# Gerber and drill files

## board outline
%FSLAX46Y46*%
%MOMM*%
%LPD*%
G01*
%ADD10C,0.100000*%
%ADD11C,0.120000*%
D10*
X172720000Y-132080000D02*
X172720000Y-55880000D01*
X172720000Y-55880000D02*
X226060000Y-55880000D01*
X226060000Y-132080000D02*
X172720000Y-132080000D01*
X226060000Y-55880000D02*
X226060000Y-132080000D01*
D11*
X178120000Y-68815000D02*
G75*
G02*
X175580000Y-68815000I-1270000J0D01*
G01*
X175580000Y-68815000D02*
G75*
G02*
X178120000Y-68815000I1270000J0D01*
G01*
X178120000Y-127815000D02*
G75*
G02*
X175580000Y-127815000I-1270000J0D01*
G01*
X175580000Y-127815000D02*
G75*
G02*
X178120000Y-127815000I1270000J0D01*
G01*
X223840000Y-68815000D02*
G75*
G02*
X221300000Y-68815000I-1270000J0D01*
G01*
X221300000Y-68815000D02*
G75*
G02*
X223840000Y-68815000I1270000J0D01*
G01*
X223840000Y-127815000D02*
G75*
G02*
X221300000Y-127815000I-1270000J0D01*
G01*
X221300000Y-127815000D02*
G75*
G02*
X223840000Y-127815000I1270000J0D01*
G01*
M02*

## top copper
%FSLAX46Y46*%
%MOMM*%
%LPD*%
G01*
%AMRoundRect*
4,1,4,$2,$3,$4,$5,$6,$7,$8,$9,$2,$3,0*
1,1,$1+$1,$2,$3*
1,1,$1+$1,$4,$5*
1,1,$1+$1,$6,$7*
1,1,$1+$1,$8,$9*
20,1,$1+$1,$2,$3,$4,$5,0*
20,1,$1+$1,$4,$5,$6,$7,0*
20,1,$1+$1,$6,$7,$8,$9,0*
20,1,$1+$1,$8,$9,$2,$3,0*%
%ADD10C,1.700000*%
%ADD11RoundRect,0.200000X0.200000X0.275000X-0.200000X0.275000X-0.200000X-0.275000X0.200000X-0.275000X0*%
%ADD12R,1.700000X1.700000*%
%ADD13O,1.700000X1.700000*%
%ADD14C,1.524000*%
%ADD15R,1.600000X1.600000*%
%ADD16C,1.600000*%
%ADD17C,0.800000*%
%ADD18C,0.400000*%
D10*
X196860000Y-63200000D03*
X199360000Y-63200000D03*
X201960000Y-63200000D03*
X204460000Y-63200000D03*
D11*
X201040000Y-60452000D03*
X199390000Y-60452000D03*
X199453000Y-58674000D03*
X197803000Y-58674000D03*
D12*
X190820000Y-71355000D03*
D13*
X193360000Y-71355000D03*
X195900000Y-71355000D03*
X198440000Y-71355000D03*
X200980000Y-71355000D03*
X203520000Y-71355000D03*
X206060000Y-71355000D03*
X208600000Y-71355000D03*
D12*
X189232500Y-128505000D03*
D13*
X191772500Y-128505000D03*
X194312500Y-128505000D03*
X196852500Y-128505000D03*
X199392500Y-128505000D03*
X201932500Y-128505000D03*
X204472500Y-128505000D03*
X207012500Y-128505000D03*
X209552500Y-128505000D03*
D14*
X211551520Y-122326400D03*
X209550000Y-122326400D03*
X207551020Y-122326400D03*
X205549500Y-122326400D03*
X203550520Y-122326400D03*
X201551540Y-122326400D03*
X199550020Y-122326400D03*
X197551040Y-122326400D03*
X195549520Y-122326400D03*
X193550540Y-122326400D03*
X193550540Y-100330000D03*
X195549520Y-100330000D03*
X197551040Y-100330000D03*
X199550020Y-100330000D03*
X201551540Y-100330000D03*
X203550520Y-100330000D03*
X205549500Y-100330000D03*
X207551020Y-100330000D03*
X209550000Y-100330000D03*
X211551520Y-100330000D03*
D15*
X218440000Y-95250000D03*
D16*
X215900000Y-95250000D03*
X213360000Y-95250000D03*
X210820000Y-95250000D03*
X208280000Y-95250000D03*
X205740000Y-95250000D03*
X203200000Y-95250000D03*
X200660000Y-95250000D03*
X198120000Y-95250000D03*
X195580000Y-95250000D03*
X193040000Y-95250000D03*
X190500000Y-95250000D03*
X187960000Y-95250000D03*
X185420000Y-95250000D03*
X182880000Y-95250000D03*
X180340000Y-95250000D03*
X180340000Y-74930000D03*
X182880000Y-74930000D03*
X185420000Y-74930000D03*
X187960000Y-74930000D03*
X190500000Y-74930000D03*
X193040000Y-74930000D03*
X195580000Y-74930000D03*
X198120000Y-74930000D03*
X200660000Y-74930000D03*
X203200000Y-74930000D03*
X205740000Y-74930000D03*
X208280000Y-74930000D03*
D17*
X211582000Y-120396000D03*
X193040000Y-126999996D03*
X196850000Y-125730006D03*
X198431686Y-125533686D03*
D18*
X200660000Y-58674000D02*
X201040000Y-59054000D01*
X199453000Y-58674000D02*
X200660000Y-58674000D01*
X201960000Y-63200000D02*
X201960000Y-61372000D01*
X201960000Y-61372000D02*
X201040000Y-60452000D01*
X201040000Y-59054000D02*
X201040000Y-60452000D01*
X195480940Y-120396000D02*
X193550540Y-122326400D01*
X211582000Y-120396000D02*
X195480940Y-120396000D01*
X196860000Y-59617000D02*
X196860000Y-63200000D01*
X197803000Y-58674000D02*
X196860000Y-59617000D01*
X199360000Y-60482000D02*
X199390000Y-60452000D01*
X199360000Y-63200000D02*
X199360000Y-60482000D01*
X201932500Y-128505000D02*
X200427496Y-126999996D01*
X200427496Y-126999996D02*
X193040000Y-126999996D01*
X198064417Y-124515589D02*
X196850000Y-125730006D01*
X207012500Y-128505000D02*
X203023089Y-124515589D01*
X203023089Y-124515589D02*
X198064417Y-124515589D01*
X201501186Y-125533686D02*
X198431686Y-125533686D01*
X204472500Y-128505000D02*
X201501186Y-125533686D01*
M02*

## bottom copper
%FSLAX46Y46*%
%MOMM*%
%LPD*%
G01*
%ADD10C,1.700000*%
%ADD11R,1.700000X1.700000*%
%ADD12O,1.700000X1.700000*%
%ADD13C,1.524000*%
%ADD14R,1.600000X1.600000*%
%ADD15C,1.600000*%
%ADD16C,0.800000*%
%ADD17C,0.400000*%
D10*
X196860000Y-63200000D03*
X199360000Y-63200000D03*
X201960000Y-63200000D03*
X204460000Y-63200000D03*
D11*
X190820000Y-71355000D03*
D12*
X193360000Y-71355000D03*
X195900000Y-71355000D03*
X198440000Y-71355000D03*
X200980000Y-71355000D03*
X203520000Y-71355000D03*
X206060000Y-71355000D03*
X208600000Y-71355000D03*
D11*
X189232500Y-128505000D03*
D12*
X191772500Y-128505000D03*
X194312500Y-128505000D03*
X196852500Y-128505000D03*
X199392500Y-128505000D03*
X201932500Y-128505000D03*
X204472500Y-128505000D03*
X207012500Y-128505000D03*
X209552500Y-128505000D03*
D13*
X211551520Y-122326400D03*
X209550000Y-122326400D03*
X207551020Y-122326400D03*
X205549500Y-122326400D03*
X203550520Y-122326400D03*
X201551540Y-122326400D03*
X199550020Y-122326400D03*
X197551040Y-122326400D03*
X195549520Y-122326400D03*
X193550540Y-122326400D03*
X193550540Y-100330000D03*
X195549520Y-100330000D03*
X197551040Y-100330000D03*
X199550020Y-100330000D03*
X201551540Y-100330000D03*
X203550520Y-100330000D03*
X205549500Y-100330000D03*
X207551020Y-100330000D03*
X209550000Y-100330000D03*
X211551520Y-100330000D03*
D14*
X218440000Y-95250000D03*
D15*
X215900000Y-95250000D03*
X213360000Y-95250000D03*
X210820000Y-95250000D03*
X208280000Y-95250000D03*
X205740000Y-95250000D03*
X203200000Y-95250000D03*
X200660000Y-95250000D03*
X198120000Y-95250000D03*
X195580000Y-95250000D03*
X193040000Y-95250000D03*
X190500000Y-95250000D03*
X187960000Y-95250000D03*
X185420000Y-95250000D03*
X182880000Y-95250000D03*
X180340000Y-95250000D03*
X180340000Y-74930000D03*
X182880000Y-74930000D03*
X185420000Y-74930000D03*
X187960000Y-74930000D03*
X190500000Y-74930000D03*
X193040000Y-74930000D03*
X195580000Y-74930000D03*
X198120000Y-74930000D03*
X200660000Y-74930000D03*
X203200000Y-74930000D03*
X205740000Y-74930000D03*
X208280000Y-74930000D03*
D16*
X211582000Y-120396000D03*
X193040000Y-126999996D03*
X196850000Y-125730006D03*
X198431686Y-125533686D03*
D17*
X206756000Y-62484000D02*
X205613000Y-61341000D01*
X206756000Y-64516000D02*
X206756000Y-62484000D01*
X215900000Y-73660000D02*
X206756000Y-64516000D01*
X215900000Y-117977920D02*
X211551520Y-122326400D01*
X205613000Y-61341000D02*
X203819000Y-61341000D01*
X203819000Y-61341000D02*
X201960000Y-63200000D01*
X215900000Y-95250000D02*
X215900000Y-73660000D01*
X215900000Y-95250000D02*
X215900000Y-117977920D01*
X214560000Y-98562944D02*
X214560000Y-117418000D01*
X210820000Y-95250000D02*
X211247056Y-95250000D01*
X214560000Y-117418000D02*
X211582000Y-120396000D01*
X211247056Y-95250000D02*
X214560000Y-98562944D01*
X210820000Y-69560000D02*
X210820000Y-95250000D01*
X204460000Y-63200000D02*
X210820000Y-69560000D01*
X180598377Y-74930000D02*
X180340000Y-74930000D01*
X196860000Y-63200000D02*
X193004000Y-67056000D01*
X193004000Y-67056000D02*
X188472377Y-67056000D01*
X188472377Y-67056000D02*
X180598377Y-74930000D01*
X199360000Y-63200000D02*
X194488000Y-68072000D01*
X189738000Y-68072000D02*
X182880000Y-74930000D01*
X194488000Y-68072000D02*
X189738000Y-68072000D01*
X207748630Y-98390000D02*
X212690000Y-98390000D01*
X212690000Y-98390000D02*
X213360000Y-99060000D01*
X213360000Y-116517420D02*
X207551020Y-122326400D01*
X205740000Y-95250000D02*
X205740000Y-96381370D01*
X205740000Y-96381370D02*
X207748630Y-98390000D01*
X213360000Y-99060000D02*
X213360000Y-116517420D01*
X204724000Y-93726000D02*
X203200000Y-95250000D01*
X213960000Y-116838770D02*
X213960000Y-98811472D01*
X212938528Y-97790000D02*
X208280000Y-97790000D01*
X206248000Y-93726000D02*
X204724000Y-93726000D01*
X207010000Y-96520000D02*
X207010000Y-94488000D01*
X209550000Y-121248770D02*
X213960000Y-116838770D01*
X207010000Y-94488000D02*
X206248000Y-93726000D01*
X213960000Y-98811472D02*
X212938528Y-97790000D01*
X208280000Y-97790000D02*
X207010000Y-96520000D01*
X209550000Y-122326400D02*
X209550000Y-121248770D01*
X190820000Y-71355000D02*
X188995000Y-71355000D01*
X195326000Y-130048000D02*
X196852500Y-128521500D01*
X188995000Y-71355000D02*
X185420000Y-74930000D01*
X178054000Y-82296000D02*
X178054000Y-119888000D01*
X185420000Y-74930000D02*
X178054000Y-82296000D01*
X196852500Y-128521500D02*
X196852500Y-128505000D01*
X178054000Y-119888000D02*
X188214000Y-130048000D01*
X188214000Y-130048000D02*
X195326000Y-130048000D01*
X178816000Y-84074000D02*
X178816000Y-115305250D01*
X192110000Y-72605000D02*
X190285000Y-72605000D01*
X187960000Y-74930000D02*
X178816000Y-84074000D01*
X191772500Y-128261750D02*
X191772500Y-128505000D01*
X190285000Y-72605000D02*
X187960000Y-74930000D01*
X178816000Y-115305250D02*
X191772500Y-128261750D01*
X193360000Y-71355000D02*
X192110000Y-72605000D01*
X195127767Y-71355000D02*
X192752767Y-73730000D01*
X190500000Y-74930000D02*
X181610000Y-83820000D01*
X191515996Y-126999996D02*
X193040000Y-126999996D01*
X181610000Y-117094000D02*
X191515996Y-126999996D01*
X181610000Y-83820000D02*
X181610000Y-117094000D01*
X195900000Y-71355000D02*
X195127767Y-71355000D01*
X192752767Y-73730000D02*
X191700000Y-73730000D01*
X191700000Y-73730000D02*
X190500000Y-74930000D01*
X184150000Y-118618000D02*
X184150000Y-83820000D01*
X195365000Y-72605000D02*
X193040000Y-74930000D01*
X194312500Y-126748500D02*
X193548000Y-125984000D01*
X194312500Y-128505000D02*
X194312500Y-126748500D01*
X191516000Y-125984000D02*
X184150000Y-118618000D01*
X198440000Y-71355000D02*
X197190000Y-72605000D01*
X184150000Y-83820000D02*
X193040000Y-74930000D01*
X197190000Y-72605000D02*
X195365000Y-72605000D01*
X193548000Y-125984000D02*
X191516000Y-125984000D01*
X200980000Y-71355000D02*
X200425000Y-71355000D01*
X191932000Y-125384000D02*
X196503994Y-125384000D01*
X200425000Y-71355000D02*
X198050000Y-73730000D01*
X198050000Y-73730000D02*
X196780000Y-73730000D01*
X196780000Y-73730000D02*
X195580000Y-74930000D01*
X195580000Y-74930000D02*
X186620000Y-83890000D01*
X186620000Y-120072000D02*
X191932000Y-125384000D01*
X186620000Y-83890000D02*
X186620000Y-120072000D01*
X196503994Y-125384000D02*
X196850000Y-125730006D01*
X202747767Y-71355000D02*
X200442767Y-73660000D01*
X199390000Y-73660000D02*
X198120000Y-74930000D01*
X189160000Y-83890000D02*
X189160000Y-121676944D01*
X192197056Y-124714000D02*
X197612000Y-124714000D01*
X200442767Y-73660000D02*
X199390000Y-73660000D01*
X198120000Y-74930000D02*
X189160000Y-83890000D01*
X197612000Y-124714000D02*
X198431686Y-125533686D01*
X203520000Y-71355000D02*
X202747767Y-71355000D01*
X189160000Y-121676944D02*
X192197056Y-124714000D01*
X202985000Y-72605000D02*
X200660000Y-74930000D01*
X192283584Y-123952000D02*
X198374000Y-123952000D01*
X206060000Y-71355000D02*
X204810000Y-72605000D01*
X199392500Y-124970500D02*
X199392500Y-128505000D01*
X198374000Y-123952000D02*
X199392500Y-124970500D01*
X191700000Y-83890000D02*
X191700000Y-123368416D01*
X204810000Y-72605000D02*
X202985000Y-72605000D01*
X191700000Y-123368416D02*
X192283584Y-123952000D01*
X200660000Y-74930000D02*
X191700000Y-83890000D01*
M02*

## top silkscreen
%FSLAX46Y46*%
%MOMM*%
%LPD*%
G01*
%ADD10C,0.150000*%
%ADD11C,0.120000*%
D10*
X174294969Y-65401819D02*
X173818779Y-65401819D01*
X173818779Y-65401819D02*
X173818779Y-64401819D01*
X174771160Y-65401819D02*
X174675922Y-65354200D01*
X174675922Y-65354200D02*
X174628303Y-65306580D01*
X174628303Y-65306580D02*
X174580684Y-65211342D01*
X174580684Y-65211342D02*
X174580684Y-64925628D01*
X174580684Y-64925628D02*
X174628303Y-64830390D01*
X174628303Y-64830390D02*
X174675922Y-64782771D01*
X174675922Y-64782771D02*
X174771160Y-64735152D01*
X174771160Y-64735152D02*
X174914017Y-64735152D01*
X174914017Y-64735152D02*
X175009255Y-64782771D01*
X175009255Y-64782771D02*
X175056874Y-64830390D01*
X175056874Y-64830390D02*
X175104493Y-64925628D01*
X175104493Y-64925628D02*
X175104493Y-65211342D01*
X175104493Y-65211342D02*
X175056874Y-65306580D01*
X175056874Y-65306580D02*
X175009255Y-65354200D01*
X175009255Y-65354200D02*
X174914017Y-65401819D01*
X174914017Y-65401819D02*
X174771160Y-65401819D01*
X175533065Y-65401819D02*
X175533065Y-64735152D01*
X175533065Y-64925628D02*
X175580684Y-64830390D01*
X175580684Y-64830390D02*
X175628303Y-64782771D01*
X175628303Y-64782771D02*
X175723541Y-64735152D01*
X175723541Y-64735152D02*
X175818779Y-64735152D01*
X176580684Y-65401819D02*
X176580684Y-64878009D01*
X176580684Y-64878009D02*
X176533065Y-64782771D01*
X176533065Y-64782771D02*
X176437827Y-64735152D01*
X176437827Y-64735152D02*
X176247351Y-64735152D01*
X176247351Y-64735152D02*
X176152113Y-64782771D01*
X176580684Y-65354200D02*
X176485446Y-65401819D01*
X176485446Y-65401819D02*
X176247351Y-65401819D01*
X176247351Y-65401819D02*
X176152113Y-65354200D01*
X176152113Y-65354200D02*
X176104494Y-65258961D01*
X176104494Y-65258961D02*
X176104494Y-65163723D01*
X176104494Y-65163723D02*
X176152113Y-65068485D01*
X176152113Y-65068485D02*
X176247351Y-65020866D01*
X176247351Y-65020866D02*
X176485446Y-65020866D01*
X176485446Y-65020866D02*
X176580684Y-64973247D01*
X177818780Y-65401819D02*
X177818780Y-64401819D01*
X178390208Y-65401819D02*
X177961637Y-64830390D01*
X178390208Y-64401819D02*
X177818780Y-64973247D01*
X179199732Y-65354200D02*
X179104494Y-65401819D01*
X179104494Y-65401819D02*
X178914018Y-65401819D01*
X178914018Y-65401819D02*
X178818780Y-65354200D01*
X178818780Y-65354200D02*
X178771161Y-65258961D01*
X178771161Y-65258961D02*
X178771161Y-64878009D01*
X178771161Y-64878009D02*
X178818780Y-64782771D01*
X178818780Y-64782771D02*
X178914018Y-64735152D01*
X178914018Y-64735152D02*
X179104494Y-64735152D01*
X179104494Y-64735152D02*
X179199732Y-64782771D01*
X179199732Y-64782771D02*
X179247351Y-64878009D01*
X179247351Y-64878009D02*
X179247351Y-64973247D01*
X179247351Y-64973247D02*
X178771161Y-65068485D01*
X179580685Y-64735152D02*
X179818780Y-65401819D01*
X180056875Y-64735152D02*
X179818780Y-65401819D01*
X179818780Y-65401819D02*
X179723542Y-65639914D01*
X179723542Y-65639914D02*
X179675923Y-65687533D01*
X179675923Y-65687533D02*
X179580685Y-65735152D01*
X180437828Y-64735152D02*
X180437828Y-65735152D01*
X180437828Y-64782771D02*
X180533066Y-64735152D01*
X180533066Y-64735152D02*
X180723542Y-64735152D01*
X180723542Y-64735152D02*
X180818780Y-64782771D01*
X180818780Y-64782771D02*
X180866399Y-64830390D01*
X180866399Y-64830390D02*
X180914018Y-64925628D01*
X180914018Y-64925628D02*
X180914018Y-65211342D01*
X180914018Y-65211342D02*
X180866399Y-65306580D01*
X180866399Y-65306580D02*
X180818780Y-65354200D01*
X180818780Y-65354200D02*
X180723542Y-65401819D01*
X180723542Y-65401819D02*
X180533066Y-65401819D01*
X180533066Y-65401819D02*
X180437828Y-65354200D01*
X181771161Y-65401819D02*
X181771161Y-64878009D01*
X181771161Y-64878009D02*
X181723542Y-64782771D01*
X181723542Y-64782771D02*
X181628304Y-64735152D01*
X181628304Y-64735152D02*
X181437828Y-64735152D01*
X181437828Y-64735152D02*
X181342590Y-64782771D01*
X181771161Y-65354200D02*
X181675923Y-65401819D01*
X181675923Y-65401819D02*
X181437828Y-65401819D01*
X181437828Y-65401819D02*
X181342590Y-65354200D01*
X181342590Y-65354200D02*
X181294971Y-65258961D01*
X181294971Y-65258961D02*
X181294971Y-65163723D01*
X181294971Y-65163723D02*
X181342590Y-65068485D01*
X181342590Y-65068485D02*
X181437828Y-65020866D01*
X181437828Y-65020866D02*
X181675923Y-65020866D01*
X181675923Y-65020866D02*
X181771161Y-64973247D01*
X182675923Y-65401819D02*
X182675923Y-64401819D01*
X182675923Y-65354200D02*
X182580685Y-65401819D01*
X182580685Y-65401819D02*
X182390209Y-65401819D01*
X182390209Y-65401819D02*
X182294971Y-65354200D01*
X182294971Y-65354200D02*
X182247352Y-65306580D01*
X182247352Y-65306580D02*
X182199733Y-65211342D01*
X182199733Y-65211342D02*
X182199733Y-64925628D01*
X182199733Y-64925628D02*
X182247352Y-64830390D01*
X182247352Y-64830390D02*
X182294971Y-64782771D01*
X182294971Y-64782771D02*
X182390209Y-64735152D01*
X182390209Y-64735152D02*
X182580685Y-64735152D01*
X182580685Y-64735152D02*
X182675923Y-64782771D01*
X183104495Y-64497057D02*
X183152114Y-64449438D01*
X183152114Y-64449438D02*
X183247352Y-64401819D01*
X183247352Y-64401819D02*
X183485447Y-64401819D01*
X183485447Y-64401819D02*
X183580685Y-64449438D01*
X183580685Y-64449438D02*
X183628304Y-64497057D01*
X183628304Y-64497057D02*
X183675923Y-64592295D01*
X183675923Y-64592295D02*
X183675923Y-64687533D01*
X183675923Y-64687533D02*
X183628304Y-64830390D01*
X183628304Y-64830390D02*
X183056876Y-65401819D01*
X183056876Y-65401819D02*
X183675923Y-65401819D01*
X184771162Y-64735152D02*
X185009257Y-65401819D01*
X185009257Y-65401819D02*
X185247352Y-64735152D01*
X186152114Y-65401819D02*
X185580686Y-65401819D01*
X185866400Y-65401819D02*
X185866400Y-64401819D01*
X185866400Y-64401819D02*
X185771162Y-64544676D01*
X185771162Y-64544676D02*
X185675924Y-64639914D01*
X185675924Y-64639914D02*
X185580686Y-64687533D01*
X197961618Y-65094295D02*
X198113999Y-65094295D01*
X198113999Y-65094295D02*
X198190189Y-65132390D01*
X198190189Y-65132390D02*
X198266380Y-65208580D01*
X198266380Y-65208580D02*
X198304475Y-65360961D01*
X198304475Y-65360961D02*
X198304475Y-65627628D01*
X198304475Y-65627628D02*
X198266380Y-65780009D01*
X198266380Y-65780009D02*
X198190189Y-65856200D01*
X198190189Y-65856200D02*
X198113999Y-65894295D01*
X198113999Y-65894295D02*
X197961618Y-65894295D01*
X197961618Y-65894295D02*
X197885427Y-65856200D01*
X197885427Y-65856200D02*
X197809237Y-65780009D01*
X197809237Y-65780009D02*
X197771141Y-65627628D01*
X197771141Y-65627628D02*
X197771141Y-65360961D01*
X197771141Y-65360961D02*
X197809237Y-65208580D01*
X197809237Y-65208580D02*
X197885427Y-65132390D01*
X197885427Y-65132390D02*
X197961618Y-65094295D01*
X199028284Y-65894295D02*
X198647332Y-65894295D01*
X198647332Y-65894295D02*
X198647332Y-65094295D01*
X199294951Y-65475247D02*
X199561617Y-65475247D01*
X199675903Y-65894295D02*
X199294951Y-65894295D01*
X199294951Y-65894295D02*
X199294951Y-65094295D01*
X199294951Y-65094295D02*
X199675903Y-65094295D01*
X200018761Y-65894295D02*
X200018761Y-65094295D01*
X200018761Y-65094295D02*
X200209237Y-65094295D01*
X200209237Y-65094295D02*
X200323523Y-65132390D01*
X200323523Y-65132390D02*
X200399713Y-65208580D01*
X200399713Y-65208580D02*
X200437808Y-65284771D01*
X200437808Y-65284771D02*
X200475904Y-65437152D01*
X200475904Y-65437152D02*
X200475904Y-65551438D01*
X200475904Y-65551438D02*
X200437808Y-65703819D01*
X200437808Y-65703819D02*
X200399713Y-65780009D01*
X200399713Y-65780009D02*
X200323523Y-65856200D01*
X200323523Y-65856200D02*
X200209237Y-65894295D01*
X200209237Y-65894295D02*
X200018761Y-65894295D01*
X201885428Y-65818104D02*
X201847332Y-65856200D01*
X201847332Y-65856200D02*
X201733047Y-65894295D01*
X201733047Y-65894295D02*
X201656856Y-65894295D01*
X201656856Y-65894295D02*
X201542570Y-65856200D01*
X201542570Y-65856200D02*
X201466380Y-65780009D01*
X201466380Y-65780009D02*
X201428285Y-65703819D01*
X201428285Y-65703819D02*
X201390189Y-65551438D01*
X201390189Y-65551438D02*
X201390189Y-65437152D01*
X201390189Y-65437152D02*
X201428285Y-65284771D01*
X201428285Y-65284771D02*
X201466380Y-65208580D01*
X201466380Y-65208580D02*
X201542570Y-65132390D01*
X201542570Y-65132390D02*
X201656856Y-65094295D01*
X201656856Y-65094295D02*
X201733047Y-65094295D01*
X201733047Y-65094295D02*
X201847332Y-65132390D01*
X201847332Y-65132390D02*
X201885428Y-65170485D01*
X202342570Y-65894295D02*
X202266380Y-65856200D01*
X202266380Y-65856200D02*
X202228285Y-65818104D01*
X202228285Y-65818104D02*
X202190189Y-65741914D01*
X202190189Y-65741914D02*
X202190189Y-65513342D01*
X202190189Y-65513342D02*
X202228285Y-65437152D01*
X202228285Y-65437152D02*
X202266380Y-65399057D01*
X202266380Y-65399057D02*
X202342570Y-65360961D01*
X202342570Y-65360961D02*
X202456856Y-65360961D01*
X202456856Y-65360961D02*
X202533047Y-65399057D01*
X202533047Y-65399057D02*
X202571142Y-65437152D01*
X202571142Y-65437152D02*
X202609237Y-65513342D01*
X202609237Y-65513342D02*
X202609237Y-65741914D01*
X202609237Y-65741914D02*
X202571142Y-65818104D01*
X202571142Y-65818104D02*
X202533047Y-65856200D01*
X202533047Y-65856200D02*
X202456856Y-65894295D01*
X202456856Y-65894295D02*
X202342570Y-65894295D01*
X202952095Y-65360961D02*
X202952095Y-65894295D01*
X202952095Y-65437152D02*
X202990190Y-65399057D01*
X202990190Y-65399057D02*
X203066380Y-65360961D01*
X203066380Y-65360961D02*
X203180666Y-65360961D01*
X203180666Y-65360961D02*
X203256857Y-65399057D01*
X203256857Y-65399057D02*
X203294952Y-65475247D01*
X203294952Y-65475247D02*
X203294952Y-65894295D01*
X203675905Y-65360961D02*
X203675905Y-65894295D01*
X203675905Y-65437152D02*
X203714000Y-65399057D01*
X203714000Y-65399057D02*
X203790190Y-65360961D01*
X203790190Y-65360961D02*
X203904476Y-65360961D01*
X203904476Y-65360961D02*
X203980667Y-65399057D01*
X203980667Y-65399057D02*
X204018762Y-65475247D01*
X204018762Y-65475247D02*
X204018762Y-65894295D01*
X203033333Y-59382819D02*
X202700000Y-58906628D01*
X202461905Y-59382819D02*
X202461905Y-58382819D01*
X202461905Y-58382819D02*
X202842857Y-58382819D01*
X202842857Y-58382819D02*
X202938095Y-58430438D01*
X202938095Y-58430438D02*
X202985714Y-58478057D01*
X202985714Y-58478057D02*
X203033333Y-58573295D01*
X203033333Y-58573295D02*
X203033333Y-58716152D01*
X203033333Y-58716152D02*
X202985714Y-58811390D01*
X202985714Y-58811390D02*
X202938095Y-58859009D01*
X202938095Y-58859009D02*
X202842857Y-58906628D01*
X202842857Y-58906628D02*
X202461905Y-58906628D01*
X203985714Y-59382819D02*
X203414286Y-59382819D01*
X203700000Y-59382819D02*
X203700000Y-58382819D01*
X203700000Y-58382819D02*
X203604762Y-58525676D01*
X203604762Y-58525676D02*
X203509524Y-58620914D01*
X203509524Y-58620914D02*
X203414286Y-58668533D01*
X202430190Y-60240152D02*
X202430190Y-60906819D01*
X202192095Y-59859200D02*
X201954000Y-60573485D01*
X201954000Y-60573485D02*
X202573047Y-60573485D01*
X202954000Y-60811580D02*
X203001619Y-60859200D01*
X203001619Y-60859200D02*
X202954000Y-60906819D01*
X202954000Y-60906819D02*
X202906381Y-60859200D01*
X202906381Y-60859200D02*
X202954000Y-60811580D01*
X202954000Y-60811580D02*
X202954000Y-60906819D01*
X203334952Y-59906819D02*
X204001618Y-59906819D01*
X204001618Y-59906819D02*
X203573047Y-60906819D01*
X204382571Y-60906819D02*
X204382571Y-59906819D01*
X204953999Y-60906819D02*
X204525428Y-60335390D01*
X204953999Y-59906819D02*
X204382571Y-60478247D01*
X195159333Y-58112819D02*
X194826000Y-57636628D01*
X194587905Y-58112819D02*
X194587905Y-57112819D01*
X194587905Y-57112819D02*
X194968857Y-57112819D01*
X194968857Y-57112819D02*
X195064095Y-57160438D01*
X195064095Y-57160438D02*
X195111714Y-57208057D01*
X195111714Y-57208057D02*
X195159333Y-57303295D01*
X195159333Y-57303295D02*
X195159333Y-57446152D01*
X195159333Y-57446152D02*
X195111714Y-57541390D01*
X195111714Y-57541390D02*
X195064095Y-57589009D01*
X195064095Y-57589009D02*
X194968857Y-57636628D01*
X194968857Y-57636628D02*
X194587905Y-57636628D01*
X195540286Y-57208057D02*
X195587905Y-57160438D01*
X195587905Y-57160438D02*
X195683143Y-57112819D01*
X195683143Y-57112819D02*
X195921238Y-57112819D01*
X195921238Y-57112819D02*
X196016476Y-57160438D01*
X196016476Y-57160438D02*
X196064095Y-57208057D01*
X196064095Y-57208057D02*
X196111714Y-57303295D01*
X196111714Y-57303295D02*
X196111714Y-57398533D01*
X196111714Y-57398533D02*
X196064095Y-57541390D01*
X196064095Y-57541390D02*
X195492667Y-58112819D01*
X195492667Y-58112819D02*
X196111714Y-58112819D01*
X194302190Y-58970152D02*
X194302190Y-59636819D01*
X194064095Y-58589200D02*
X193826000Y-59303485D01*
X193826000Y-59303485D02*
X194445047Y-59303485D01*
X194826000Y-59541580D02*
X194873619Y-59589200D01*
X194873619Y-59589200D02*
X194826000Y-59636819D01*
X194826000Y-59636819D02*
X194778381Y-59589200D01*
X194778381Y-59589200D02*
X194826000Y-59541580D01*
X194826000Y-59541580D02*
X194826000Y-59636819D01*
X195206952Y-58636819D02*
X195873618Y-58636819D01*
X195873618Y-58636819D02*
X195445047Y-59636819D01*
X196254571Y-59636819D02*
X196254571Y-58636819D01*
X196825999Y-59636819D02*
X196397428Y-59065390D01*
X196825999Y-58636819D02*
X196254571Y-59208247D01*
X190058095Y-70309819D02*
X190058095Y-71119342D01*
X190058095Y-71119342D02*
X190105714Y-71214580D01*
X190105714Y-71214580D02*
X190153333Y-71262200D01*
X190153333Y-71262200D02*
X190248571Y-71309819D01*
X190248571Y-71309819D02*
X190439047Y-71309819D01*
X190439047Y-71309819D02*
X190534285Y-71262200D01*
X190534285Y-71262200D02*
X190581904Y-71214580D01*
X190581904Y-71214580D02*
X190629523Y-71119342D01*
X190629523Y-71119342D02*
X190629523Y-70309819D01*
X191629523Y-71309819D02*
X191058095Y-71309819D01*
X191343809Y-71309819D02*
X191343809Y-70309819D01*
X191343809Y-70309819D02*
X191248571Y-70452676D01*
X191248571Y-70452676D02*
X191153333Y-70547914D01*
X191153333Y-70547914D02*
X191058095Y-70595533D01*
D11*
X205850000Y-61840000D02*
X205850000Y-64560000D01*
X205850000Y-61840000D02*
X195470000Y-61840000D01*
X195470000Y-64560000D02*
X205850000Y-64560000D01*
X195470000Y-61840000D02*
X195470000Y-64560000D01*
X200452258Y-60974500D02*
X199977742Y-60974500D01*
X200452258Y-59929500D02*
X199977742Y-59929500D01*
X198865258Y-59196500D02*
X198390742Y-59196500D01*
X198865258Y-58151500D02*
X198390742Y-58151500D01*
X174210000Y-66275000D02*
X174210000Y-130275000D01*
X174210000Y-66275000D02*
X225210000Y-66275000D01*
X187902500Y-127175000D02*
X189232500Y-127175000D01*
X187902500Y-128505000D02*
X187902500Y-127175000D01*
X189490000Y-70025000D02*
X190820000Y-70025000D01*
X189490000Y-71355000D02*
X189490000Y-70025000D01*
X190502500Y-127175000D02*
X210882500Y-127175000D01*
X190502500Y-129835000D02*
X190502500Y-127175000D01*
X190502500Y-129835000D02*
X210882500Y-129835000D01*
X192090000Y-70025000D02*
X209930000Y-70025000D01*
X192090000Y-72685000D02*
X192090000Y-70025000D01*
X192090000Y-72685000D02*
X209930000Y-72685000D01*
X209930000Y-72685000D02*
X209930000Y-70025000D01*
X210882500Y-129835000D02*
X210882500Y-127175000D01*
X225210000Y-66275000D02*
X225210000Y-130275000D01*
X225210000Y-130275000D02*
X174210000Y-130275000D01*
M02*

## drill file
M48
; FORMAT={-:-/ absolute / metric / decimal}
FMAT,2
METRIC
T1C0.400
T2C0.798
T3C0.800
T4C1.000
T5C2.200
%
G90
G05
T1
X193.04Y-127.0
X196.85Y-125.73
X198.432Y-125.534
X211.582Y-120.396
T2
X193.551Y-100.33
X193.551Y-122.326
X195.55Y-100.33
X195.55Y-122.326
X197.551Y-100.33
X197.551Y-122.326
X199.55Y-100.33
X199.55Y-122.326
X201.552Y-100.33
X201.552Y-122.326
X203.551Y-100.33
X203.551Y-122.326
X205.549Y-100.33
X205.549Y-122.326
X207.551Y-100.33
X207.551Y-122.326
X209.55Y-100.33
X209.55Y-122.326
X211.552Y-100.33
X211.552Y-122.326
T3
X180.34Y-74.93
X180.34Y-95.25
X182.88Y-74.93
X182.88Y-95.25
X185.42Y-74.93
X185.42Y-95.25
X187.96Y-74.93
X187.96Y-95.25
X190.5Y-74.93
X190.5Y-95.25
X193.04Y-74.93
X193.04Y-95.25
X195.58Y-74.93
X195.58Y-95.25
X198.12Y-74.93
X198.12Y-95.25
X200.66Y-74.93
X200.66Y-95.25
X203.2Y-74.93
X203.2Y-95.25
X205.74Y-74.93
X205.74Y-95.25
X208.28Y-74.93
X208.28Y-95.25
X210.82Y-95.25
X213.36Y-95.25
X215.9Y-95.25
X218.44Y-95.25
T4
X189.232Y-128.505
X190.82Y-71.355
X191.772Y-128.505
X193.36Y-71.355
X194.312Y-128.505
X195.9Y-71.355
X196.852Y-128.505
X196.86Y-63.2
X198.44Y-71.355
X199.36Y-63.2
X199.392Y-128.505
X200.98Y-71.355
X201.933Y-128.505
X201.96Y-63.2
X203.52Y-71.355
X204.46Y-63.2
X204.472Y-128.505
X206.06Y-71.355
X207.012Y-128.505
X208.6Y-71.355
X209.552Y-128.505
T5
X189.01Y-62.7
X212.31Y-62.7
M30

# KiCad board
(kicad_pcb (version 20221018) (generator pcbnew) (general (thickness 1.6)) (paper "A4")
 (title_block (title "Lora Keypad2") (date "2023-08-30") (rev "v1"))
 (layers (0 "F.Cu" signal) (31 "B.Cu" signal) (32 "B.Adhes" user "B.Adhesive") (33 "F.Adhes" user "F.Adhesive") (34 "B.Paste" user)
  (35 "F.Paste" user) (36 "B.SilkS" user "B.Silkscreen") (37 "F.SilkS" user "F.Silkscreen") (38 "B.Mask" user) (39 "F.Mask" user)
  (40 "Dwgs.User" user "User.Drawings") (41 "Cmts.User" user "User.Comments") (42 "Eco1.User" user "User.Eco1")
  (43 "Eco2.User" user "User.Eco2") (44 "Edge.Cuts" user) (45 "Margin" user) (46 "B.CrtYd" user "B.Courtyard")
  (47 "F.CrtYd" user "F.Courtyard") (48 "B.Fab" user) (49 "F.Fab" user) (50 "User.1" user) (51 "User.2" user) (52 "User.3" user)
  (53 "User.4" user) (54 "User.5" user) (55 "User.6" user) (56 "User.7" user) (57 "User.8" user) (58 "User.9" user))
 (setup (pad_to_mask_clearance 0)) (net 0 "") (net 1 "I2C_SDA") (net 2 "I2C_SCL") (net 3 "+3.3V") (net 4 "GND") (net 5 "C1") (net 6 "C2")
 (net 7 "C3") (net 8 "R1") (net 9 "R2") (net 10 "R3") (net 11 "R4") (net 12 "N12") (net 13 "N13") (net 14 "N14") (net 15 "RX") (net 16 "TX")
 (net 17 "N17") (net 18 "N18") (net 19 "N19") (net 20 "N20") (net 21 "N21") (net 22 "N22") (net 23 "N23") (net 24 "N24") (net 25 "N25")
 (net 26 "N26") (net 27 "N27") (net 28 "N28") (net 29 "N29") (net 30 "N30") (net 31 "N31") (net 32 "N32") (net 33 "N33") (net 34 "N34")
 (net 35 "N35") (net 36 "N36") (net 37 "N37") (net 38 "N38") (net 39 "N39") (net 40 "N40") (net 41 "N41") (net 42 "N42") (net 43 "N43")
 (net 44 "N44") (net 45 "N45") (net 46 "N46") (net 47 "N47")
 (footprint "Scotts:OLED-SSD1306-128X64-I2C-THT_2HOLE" (layer "F.Cu") (at 200.66 63.2 180)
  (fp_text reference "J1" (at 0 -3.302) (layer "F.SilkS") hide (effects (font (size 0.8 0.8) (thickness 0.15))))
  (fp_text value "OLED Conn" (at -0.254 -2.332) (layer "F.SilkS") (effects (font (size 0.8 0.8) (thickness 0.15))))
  (fp_line (start -5.19 1.36) (end -5.19 -1.36) (stroke (width 0.12) (type solid)) (layer "F.SilkS"))
  (fp_line (start -5.19 1.36) (end 5.19 1.36) (stroke (width 0.12) (type solid)) (layer "F.SilkS"))
  (fp_line (start 5.19 -1.36) (end -5.19 -1.36) (stroke (width 0.12) (type solid)) (layer "F.SilkS"))
  (fp_line (start 5.19 1.36) (end 5.19 -1.36) (stroke (width 0.12) (type solid)) (layer "F.SilkS"))
  (pad "" np_thru_hole circle (at -11.65 0.5 180) (size 2.2 2.2) (drill 2.2) (layers "*.Cu" "*.Mask") (solder_mask_margin 1.4)
   (clearance 1.4))
  (pad "" np_thru_hole circle (at 11.65 0.5 180) (size 2.2 2.2) (drill 2.2) (layers "*.Cu" "*.Mask") (solder_mask_margin 1.4)
   (clearance 1.4))
  (pad "1" thru_hole circle (at 3.8 0 180) (size 1.7 1.7) (drill 1) (layers "*.Cu" "*.Mask") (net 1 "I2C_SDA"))
  (pad "2" thru_hole circle (at 1.3 0 180) (size 1.7 1.7) (drill 1) (layers "*.Cu" "*.Mask") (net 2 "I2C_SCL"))
  (pad "3" thru_hole circle (at -1.3 0 180) (size 1.7 1.7) (drill 1) (layers "*.Cu" "*.Mask") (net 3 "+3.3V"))
  (pad "4" thru_hole circle (at -3.8 0 180) (size 1.7 1.7) (drill 1) (layers "*.Cu" "*.Mask") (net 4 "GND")))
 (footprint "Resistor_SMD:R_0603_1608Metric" (layer "F.Cu") (at 200.215 60.452 180)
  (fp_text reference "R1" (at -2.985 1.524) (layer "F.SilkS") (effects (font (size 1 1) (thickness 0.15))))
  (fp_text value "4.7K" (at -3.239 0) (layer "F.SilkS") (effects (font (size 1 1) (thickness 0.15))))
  (fp_line (start -0.237258 -0.5225) (end 0.237258 -0.5225) (stroke (width 0.12) (type solid)) (layer "F.SilkS"))
  (fp_line (start -0.237258 0.5225) (end 0.237258 0.5225) (stroke (width 0.12) (type solid)) (layer "F.SilkS"))
  (pad "1" smd roundrect (at -0.825 0 180) (size 0.8 0.95) (layers "F.Cu" "F.Paste" "F.Mask") (roundrect_rratio 0.25) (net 3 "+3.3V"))
  (pad "2" smd roundrect (at 0.825 0 180) (size 0.8 0.95) (layers "F.Cu" "F.Paste" "F.Mask") (roundrect_rratio 0.25) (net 2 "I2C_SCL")))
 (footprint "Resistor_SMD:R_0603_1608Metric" (layer "F.Cu") (at 198.628 58.674 180)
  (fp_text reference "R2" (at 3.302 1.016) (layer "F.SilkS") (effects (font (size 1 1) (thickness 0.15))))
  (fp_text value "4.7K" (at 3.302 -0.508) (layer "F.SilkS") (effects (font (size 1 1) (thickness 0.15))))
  (fp_line (start -0.237258 -0.5225) (end 0.237258 -0.5225) (stroke (width 0.12) (type solid)) (layer "F.SilkS"))
  (fp_line (start -0.237258 0.5225) (end 0.237258 0.5225) (stroke (width 0.12) (type solid)) (layer "F.SilkS"))
  (pad "1" smd roundrect (at -0.825 0 180) (size 0.8 0.95) (layers "F.Cu" "F.Paste" "F.Mask") (roundrect_rratio 0.25) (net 3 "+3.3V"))
  (pad "2" smd roundrect (at 0.825 0 180) (size 0.8 0.95) (layers "F.Cu" "F.Paste" "F.Mask") (roundrect_rratio 0.25) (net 1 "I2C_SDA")))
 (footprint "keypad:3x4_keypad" (layer "F.Cu") (at 190.82 71.355)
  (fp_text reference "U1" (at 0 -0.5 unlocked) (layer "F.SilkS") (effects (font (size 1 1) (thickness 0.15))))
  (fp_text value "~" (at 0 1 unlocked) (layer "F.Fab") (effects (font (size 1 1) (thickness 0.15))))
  (fp_line (start -16.61 -5.08) (end -16.61 58.92) (stroke (width 0.12) (type solid)) (layer "F.SilkS"))
  (fp_line (start -16.61 -5.08) (end 34.39 -5.08) (stroke (width 0.12) (type solid)) (layer "F.SilkS"))
  (fp_line (start -2.9175 55.82) (end -1.5875 55.82) (stroke (width 0.12) (type solid)) (layer "F.SilkS"))
  (fp_line (start -2.9175 57.15) (end -2.9175 55.82) (stroke (width 0.12) (type solid)) (layer "F.SilkS"))
  (fp_line (start -1.33 -1.33) (end 0 -1.33) (stroke (width 0.12) (type solid)) (layer "F.SilkS"))
  (fp_line (start -1.33 0) (end -1.33 -1.33) (stroke (width 0.12) (type solid)) (layer "F.SilkS"))
  (fp_line (start -0.3175 55.82) (end 20.0625 55.82) (stroke (width 0.12) (type solid)) (layer "F.SilkS"))
  (fp_line (start -0.3175 58.48) (end -0.3175 55.82) (stroke (width 0.12) (type solid)) (layer "F.SilkS"))
  (fp_line (start -0.3175 58.48) (end 20.0625 58.48) (stroke (width 0.12) (type solid)) (layer "F.SilkS"))
  (fp_line (start 1.27 -1.33) (end 19.11 -1.33) (stroke (width 0.12) (type solid)) (layer "F.SilkS"))
  (fp_line (start 1.27 1.33) (end 1.27 -1.33) (stroke (width 0.12) (type solid)) (layer "F.SilkS"))
  (fp_line (start 1.27 1.33) (end 19.11 1.33) (stroke (width 0.12) (type solid)) (layer "F.SilkS"))
  (fp_line (start 19.11 1.33) (end 19.11 -1.33) (stroke (width 0.12) (type solid)) (layer "F.SilkS"))
  (fp_line (start 20.0625 58.48) (end 20.0625 55.82) (stroke (width 0.12) (type solid)) (layer "F.SilkS"))
  (fp_line (start 34.39 -5.08) (end 34.39 58.92) (stroke (width 0.12) (type solid)) (layer "F.SilkS"))
  (fp_line (start 34.39 58.92) (end -16.61 58.92) (stroke (width 0.12) (type solid)) (layer "F.SilkS"))
  (fp_circle (center -13.97 -2.54) (end -13.97 -3.81) (stroke (width 0.12) (type default)) (fill none) (layer "Edge.Cuts"))
  (fp_circle (center -13.97 56.46) (end -12.7 56.46) (stroke (width 0.12) (type default)) (fill none) (layer "Edge.Cuts"))
  (fp_circle (center 31.75 -2.54) (end 30.48 -2.54) (stroke (width 0.12) (type default)) (fill none) (layer "Edge.Cuts"))
  (fp_circle (center 31.75 56.46) (end 33.02 56.46) (stroke (width 0.12) (type default)) (fill none) (layer "Edge.Cuts"))
  (pad "A1" thru_hole rect (at 0 0 90) (size 1.7 1.7) (drill 1) (layers "*.Cu" "*.Mask") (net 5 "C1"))
  (pad "A2" thru_hole oval (at 2.54 0 90) (size 1.7 1.7) (drill 1) (layers "*.Cu" "*.Mask") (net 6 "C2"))
  (pad "A3" thru_hole oval (at 5.08 0 90) (size 1.7 1.7) (drill 1) (layers "*.Cu" "*.Mask") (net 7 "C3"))
  (pad "A4" thru_hole oval (at 7.62 0 90) (size 1.7 1.7) (drill 1) (layers "*.Cu" "*.Mask") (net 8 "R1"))
  (pad "A5" thru_hole oval (at 10.16 0 90) (size 1.7 1.7) (drill 1) (layers "*.Cu" "*.Mask") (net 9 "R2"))
  (pad "A6" thru_hole oval (at 12.7 0 90) (size 1.7 1.7) (drill 1) (layers "*.Cu" "*.Mask") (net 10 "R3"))
  (pad "A7" thru_hole oval (at 15.24 0 90) (size 1.7 1.7) (drill 1) (layers "*.Cu" "*.Mask") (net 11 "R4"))
  (pad "A8" thru_hole oval (at 17.78 0 90) (size 1.7 1.7) (drill 1) (layers "*.Cu" "*.Mask") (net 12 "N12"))
  (pad "B1" thru_hole rect (at -1.5875 57.15 90) (size 1.7 1.7) (drill 1) (layers "*.Cu" "*.Mask") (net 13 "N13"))
  (pad "B2" thru_hole oval (at 0.9525 57.15 90) (size 1.7 1.7) (drill 1) (layers "*.Cu" "*.Mask") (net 6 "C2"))
  (pad "B3" thru_hole oval (at 3.4925 57.15 90) (size 1.7 1.7) (drill 1) (layers "*.Cu" "*.Mask") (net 8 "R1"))
  (pad "B4" thru_hole oval (at 6.0325 57.15 90) (size 1.7 1.7) (drill 1) (layers "*.Cu" "*.Mask") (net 5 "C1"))
  (pad "B5" thru_hole oval (at 8.5725 57.15 90) (size 1.7 1.7) (drill 1) (layers "*.Cu" "*.Mask") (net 11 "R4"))
  (pad "B6" thru_hole oval (at 11.1125 57.15 90) (size 1.7 1.7) (drill 1) (layers "*.Cu" "*.Mask") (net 7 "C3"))
  (pad "B7" thru_hole oval (at 13.6525 57.15 90) (size 1.7 1.7) (drill 1) (layers "*.Cu" "*.Mask") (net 10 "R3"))
  (pad "B8" thru_hole oval (at 16.1925 57.15 90) (size 1.7 1.7) (drill 1) (layers "*.Cu" "*.Mask") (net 9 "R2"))
  (pad "B9" thru_hole oval (at 18.7325 57.15 90) (size 1.7 1.7) (drill 1) (layers "*.Cu" "*.Mask") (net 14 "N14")))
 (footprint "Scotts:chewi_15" (layer "B.Cu") (at 200.406 82.804 180)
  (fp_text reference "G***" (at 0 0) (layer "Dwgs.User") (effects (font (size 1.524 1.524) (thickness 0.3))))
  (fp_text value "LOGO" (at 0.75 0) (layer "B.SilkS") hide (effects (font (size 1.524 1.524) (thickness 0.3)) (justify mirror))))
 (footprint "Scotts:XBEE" (layer "B.Cu") (at 191.55156 111.3282 90)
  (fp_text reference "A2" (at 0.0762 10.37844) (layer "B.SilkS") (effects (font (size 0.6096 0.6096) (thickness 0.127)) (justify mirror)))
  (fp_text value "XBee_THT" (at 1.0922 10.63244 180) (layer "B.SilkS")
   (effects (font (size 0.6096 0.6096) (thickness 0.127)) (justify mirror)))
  (pad "1" thru_hole circle (at -10.9982 19.99996 90) (size 1.524 1.524) (drill 0.79756) (layers "*.Cu" "*.Mask") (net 3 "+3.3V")
   (solder_mask_margin 0.1016))
  (pad "2" thru_hole circle (at -10.9982 17.99844 90) (size 1.524 1.524) (drill 0.79756) (layers "*.Cu" "*.Mask") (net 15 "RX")
   (solder_mask_margin 0.1016))
  (pad "3" thru_hole circle (at -10.9982 15.99946 90) (size 1.524 1.524) (drill 0.79756) (layers "*.Cu" "*.Mask") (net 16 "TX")
   (solder_mask_margin 0.1016))
  (pad "4" thru_hole circle (at -10.9982 13.99794 90) (size 1.524 1.524) (drill 0.79756) (layers "*.Cu" "*.Mask") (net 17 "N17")
   (solder_mask_margin 0.1016))
  (pad "5" thru_hole circle (at -10.9982 11.99896 90) (size 1.524 1.524) (drill 0.79756) (layers "*.Cu" "*.Mask") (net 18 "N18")
   (solder_mask_margin 0.1016))
  (pad "6" thru_hole circle (at -10.9982 9.99998 90) (size 1.524 1.524) (drill 0.79756) (layers "*.Cu" "*.Mask") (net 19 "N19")
   (solder_mask_margin 0.1016))
  (pad "7" thru_hole circle (at -10.9982 7.99846 90) (size 1.524 1.524) (drill 0.79756) (layers "*.Cu" "*.Mask") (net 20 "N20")
   (solder_mask_margin 0.1016))
  (pad "8" thru_hole circle (at -10.9982 5.99948 90) (size 1.524 1.524) (drill 0.79756) (layers "*.Cu" "*.Mask") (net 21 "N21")
   (solder_mask_margin 0.1016))
  (pad "9" thru_hole circle (at -10.9982 3.99796 90) (size 1.524 1.524) (drill 0.79756) (layers "*.Cu" "*.Mask") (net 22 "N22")
   (solder_mask_margin 0.1016))
  (pad "10" thru_hole circle (at -10.9982 1.99898 90) (size 1.524 1.524) (drill 0.79756) (layers "*.Cu" "*.Mask") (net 4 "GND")
   (solder_mask_margin 0.1016))
  (pad "11" thru_hole circle (at 10.9982 1.99898 90) (size 1.524 1.524) (drill 0.79756) (layers "*.Cu" "*.Mask") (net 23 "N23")
   (solder_mask_margin 0.1016))
  (pad "12" thru_hole circle (at 10.9982 3.99796 90) (size 1.524 1.524) (drill 0.79756) (layers "*.Cu" "*.Mask") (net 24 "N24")
   (solder_mask_margin 0.1016))
  (pad "13" thru_hole circle (at 10.9982 5.99948 90) (size 1.524 1.524) (drill 0.79756) (layers "*.Cu" "*.Mask") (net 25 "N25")
   (solder_mask_margin 0.1016))
  (pad "14" thru_hole circle (at 10.9982 7.99846 90) (size 1.524 1.524) (drill 0.79756) (layers "*.Cu" "*.Mask") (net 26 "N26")
   (solder_mask_margin 0.1016))
  (pad "15" thru_hole circle (at 10.9982 9.99998 90) (size 1.524 1.524) (drill 0.79756) (layers "*.Cu" "*.Mask") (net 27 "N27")
   (solder_mask_margin 0.1016))
  (pad "16" thru_hole circle (at 10.9982 11.99896 90) (size 1.524 1.524) (drill 0.79756) (layers "*.Cu" "*.Mask") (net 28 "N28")
   (solder_mask_margin 0.1016))
  (pad "17" thru_hole circle (at 10.9982 13.99794 90) (size 1.524 1.524) (drill 0.79756) (layers "*.Cu" "*.Mask") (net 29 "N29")
   (solder_mask_margin 0.1016))
  (pad "18" thru_hole circle (at 10.9982 15.99946 90) (size 1.524 1.524) (drill 0.79756) (layers "*.Cu" "*.Mask") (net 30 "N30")
   (solder_mask_margin 0.1016))
  (pad "19" thru_hole circle (at 10.9982 17.99844 90) (size 1.524 1.524) (drill 0.79756) (layers "*.Cu" "*.Mask") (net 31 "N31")
   (solder_mask_margin 0.1016))
  (pad "20" thru_hole circle (at 10.9982 19.99996 90) (size 1.524 1.524) (drill 0.79756) (layers "*.Cu" "*.Mask") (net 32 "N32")
   (solder_mask_margin 0.1016)))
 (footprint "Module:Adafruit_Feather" (layer "B.Cu") (at 218.44 95.25 90)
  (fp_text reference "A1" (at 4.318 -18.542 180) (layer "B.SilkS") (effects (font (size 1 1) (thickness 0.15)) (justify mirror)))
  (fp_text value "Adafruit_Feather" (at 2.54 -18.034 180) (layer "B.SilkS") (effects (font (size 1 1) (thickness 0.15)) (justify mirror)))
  (pad "1" thru_hole rect (at 0 0 270) (size 1.6 1.6) (drill 0.8) (layers "*.Cu" "*.Mask") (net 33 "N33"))
  (pad "2" thru_hole circle (at 0 -2.54 270) (size 1.6 1.6) (drill 0.8) (layers "*.Cu" "*.Mask") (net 3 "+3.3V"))
  (pad "3" thru_hole circle (at 0 -5.08 270) (size 1.6 1.6) (drill 0.8) (layers "*.Cu" "*.Mask") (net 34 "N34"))
  (pad "4" thru_hole circle (at 0 -7.62 270) (size 1.6 1.6) (drill 0.8) (layers "*.Cu" "*.Mask") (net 4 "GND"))
  (pad "5" thru_hole circle (at 0 -10.16 270) (size 1.6 1.6) (drill 0.8) (layers "*.Cu" "*.Mask") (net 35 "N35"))
  (pad "6" thru_hole circle (at 0 -12.7 270) (size 1.6 1.6) (drill 0.8) (layers "*.Cu" "*.Mask") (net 16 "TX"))
  (pad "7" thru_hole circle (at 0 -15.24 270) (size 1.6 1.6) (drill 0.8) (layers "*.Cu" "*.Mask") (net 15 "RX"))
  (pad "8" thru_hole circle (at 0 -17.78 270) (size 1.6 1.6) (drill 0.8) (layers "*.Cu" "*.Mask") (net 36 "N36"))
  (pad "9" thru_hole circle (at 0 -20.32 270) (size 1.6 1.6) (drill 0.8) (layers "*.Cu" "*.Mask") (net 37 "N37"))
  (pad "10" thru_hole circle (at 0 -22.86 270) (size 1.6 1.6) (drill 0.8) (layers "*.Cu" "*.Mask") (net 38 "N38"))
  (pad "11" thru_hole circle (at 0 -25.4 270) (size 1.6 1.6) (drill 0.8) (layers "*.Cu" "*.Mask") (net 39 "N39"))
  (pad "12" thru_hole circle (at 0 -27.94 270) (size 1.6 1.6) (drill 0.8) (layers "*.Cu" "*.Mask") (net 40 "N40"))
  (pad "13" thru_hole circle (at 0 -30.48 270) (size 1.6 1.6) (drill 0.8) (layers "*.Cu" "*.Mask") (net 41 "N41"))
  (pad "14" thru_hole circle (at 0 -33.02 270) (size 1.6 1.6) (drill 0.8) (layers "*.Cu" "*.Mask") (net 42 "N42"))
  (pad "15" thru_hole circle (at 0 -35.56 270) (size 1.6 1.6) (drill 0.8) (layers "*.Cu" "*.Mask") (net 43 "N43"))
  (pad "16" thru_hole circle (at 0 -38.1 270) (size 1.6 1.6) (drill 0.8) (layers "*.Cu" "*.Mask") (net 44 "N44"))
  (pad "17" thru_hole circle (at 20.32 -38.1 270) (size 1.6 1.6) (drill 0.8) (layers "*.Cu" "*.Mask") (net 1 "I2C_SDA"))
  (pad "18" thru_hole circle (at 20.32 -35.56 270) (size 1.6 1.6) (drill 0.8) (layers "*.Cu" "*.Mask") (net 2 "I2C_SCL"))
  (pad "19" thru_hole circle (at 20.32 -33.02 270) (size 1.6 1.6) (drill 0.8) (layers "*.Cu" "*.Mask") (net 5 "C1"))
  (pad "20" thru_hole circle (at 20.32 -30.48 270) (size 1.6 1.6) (drill 0.8) (layers "*.Cu" "*.Mask") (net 6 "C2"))
  (pad "21" thru_hole circle (at 20.32 -27.94 270) (size 1.6 1.6) (drill 0.8) (layers "*.Cu" "*.Mask") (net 7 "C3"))
  (pad "22" thru_hole circle (at 20.32 -25.4 270) (size 1.6 1.6) (drill 0.8) (layers "*.Cu" "*.Mask") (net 8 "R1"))
  (pad "23" thru_hole circle (at 20.32 -22.86 270) (size 1.6 1.6) (drill 0.8) (layers "*.Cu" "*.Mask") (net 9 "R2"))
  (pad "24" thru_hole circle (at 20.32 -20.32 270) (size 1.6 1.6) (drill 0.8) (layers "*.Cu" "*.Mask") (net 10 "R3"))
  (pad "25" thru_hole circle (at 20.32 -17.78 270) (size 1.6 1.6) (drill 0.8) (layers "*.Cu" "*.Mask") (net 11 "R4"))
  (pad "26" thru_hole circle (at 20.32 -15.24 270) (size 1.6 1.6) (drill 0.8) (layers "*.Cu" "*.Mask") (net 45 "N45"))
  (pad "27" thru_hole circle (at 20.32 -12.7 270) (size 1.6 1.6) (drill 0.8) (layers "*.Cu" "*.Mask") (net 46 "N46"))
  (pad "28" thru_hole circle (at 20.32 -10.16 270) (size 1.6 1.6) (drill 0.8) (layers "*.Cu" "*.Mask") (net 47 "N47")))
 (gr_line (start 172.72 132.08) (end 172.72 55.88) (stroke (width 0.1) (type default)) (layer "Edge.Cuts"))
 (gr_line (start 172.72 55.88) (end 226.06 55.88) (stroke (width 0.1) (type default)) (layer "Edge.Cuts"))
 (gr_line (start 226.06 132.08) (end 172.72 132.08) (stroke (width 0.1) (type default)) (layer "Edge.Cuts"))
 (gr_line (start 226.06 55.88) (end 226.06 132.08) (stroke (width 0.1) (type default)) (layer "Edge.Cuts"))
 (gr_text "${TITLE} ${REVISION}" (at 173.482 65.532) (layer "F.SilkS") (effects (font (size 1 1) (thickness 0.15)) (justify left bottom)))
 (segment (start 200.66 58.674) (end 201.04 59.054) (width 0.4) (layer "F.Cu") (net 3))
 (segment (start 199.453 58.674) (end 200.66 58.674) (width 0.4) (layer "F.Cu") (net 3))
 (segment (start 201.96 63.2) (end 201.96 61.372) (width 0.4) (layer "F.Cu") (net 3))
 (segment (start 201.96 61.372) (end 201.04 60.452) (width 0.4) (layer "F.Cu") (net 3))
 (segment (start 201.04 59.054) (end 201.04 60.452) (width 0.4) (layer "F.Cu") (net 3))
 (segment (start 206.756 62.484) (end 205.613 61.341) (width 0.4) (layer "B.Cu") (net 3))
 (segment (start 206.756 64.516) (end 206.756 62.484) (width 0.4) (layer "B.Cu") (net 3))
 (segment (start 215.9 73.66) (end 206.756 64.516) (width 0.4) (layer "B.Cu") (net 3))
 (segment (start 215.9 117.97792) (end 211.55152 122.3264) (width 0.4) (layer "B.Cu") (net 3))
 (segment (start 205.613 61.341) (end 203.819 61.341) (width 0.4) (layer "B.Cu") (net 3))
 (segment (start 203.819 61.341) (end 201.96 63.2) (width 0.4) (layer "B.Cu") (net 3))
 (segment (start 215.9 95.25) (end 215.9 73.66) (width 0.4) (layer "B.Cu") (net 3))
 (segment (start 215.9 95.25) (end 215.9 117.97792) (width 0.4) (layer "B.Cu") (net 3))
 (segment (start 195.48094 120.396) (end 193.55054 122.3264) (width 0.4) (layer "F.Cu") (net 4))
 (segment (start 211.582 120.396) (end 195.48094 120.396) (width 0.4) (layer "F.Cu") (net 4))
 (via (at 211.582 120.396) (size 0.8) (drill 0.4) (layers "F.Cu" "B.Cu") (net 4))
 (segment (start 214.56 98.562944) (end 214.56 117.418) (width 0.4) (layer "B.Cu") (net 4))
 (segment (start 210.82 95.25) (end 211.247056 95.25) (width 0.4) (layer "B.Cu") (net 4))
 (segment (start 214.56 117.418) (end 211.582 120.396) (width 0.4) (layer "B.Cu") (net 4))
 (segment (start 211.247056 95.25) (end 214.56 98.562944) (width 0.4) (layer "B.Cu") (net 4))
 (segment (start 210.82 69.56) (end 210.82 95.25) (width 0.4) (layer "B.Cu") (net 4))
 (segment (start 204.46 63.2) (end 210.82 69.56) (width 0.4) (layer "B.Cu") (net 4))
 (segment (start 196.86 59.617) (end 196.86 63.2) (width 0.4) (layer "F.Cu") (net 1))
 (segment (start 197.803 58.674) (end 196.86 59.617) (width 0.4) (layer "F.Cu") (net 1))
 (segment (start 180.598377 74.93) (end 180.34 74.93) (width 0.4) (layer "B.Cu") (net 1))
 (segment (start 196.86 63.2) (end 193.004 67.056) (width 0.4) (layer "B.Cu") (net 1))
 (segment (start 193.004 67.056) (end 188.472377 67.056) (width 0.4) (layer "B.Cu") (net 1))
 (segment (start 188.472377 67.056) (end 180.598377 74.93) (width 0.4) (layer "B.Cu") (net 1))
 (segment (start 199.36 60.482) (end 199.39 60.452) (width 0.4) (layer "F.Cu") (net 2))
 (segment (start 199.36 63.2) (end 199.36 60.482) (width 0.4) (layer "F.Cu") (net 2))
 (segment (start 199.36 63.2) (end 194.488 68.072) (width 0.4) (layer "B.Cu") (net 2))
 (segment (start 189.738 68.072) (end 182.88 74.93) (width 0.4) (layer "B.Cu") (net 2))
 (segment (start 194.488 68.072) (end 189.738 68.072) (width 0.4) (layer "B.Cu") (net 2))
 (segment (start 207.74863 98.39) (end 212.69 98.39) (width 0.4) (layer "B.Cu") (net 16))
 (segment (start 212.69 98.39) (end 213.36 99.06) (width 0.4) (layer "B.Cu") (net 16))
 (segment (start 213.36 116.51742) (end 207.55102 122.3264) (width 0.4) (layer "B.Cu") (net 16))
 (segment (start 205.74 95.25) (end 205.74 96.38137) (width 0.4) (layer "B.Cu") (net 16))
 (segment (start 205.74 96.38137) (end 207.74863 98.39) (width 0.4) (layer "B.Cu") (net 16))
 (segment (start 213.36 99.06) (end 213.36 116.51742) (width 0.4) (layer "B.Cu") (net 16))
 (segment (start 204.724 93.726) (end 203.2 95.25) (width 0.4) (layer "B.Cu") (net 15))
 (segment (start 213.96 116.83877) (end 213.96 98.811472) (width 0.4) (layer "B.Cu") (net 15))
 (segment (start 212.938528 97.79) (end 208.28 97.79) (width 0.4) (layer "B.Cu") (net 15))
 (segment (start 206.248 93.726) (end 204.724 93.726) (width 0.4) (layer "B.Cu") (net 15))
 (segment (start 207.01 96.52) (end 207.01 94.488) (width 0.4) (layer "B.Cu") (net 15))
 (segment (start 209.55 121.24877) (end 213.96 116.83877) (width 0.4) (layer "B.Cu") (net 15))
 (segment (start 207.01 94.488) (end 206.248 93.726) (width 0.4) (layer "B.Cu") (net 15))
 (segment (start 213.96 98.811472) (end 212.938528 97.79) (width 0.4) (layer "B.Cu") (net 15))
 (segment (start 208.28 97.79) (end 207.01 96.52) (width 0.4) (layer "B.Cu") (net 15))
 (segment (start 209.55 122.3264) (end 209.55 121.24877) (width 0.4) (layer "B.Cu") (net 15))
 (segment (start 190.82 71.355) (end 188.995 71.355) (width 0.4) (layer "B.Cu") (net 5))
 (segment (start 195.326 130.048) (end 196.8525 128.5215) (width 0.4) (layer "B.Cu") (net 5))
 (segment (start 188.995 71.355) (end 185.42 74.93) (width 0.4) (layer "B.Cu") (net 5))
 (segment (start 178.054 82.296) (end 178.054 119.888) (width 0.4) (layer "B.Cu") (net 5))
 (segment (start 185.42 74.93) (end 178.054 82.296) (width 0.4) (layer "B.Cu") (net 5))
 (segment (start 196.8525 128.5215) (end 196.8525 128.505) (width 0.4) (layer "B.Cu") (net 5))
 (segment (start 178.054 119.888) (end 188.214 130.048) (width 0.4) (layer "B.Cu") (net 5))
 (segment (start 188.214 130.048) (end 195.326 130.048) (width 0.4) (layer "B.Cu") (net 5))
 (segment (start 178.816 84.074) (end 178.816 115.30525) (width 0.4) (layer "B.Cu") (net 6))
 (segment (start 192.11 72.605) (end 190.285 72.605) (width 0.4) (layer "B.Cu") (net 6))
 (segment (start 187.96 74.93) (end 178.816 84.074) (width 0.4) (layer "B.Cu") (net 6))
 (segment (start 191.7725 128.26175) (end 191.7725 128.505) (width 0.4) (layer "B.Cu") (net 6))
 (segment (start 190.285 72.605) (end 187.96 74.93) (width 0.4) (layer "B.Cu") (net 6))
 (segment (start 178.816 115.30525) (end 191.7725 128.26175) (width 0.4) (layer "B.Cu") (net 6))
 (segment (start 193.36 71.355) (end 192.11 72.605) (width 0.4) (layer "B.Cu") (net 6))
 (segment (start 201.9325 128.505) (end 200.427496 126.999996) (width 0.4) (layer "F.Cu") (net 7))
 (segment (start 200.427496 126.999996) (end 193.04 126.999996) (width 0.4) (layer "F.Cu") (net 7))
 (via (at 193.04 126.999996) (size 0.8) (drill 0.4) (layers "F.Cu" "B.Cu") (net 7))
 (segment (start 195.127767 71.355) (end 192.752767 73.73) (width 0.4) (layer "B.Cu") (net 7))
 (segment (start 190.5 74.93) (end 181.61 83.82) (width 0.4) (layer "B.Cu") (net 7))
 (segment (start 191.515996 126.999996) (end 193.04 126.999996) (width 0.4) (layer "B.Cu") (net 7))
 (segment (start 181.61 117.094) (end 191.515996 126.999996) (width 0.4) (layer "B.Cu") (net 7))
 (segment (start 181.61 83.82) (end 181.61 117.094) (width 0.4) (layer "B.Cu") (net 7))
 (segment (start 195.9 71.355) (end 195.127767 71.355) (width 0.4) (layer "B.Cu") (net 7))
 (segment (start 192.752767 73.73) (end 191.7 73.73) (width 0.4) (layer "B.Cu") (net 7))
 (segment (start 191.7 73.73) (end 190.5 74.93) (width 0.4) (layer "B.Cu") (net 7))
 (segment (start 184.15 118.618) (end 184.15 83.82) (width 0.4) (layer "B.Cu") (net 8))
 (segment (start 195.365 72.605) (end 193.04 74.93) (width 0.4) (layer "B.Cu") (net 8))
 (segment (start 194.3125 126.7485) (end 193.548 125.984) (width 0.4) (layer "B.Cu") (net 8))
 (segment (start 194.3125 128.505) (end 194.3125 126.7485) (width 0.4) (layer "B.Cu") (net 8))
 (segment (start 191.516 125.984) (end 184.15 118.618) (width 0.4) (layer "B.Cu") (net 8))
 (segment (start 198.44 71.355) (end 197.19 72.605) (width 0.4) (layer "B.Cu") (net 8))
 (segment (start 184.15 83.82) (end 193.04 74.93) (width 0.4) (layer "B.Cu") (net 8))
 (segment (start 197.19 72.605) (end 195.365 72.605) (width 0.4) (layer "B.Cu") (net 8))
 (segment (start 193.548 125.984) (end 191.516 125.984) (width 0.4) (layer "B.Cu") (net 8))
 (segment (start 198.064417 124.515589) (end 196.85 125.730006) (width 0.4) (layer "F.Cu") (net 9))
 (segment (start 207.0125 128.505) (end 203.023089 124.515589) (width 0.4) (layer "F.Cu") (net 9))
 (segment (start 203.023089 124.515589) (end 198.064417 124.515589) (width 0.4) (layer "F.Cu") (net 9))
 (via (at 196.85 125.730006) (size 0.8) (drill 0.4) (layers "F.Cu" "B.Cu") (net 9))
 (segment (start 200.98 71.355) (end 200.425 71.355) (width 0.4) (layer "B.Cu") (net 9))
 (segment (start 191.932 125.384) (end 196.503994 125.384) (width 0.4) (layer "B.Cu") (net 9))
 (segment (start 200.425 71.355) (end 198.05 73.73) (width 0.4) (layer "B.Cu") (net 9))
 (segment (start 198.05 73.73) (end 196.78 73.73) (width 0.4) (layer "B.Cu") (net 9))
 (segment (start 196.78 73.73) (end 195.58 74.93) (width 0.4) (layer "B.Cu") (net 9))
 (segment (start 195.58 74.93) (end 186.62 83.89) (width 0.4) (layer "B.Cu") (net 9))
 (segment (start 186.62 120.072) (end 191.932 125.384) (width 0.4) (layer "B.Cu") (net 9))
 (segment (start 186.62 83.89) (end 186.62 120.072) (width 0.4) (layer "B.Cu") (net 9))
 (segment (start 196.503994 125.384) (end 196.85 125.730006) (width 0.4) (layer "B.Cu") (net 9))
 (segment (start 201.501186 125.533686) (end 198.431686 125.533686) (width 0.4) (layer "F.Cu") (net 10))
 (segment (start 204.4725 128.505) (end 201.501186 125.533686) (width 0.4) (layer "F.Cu") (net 10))
 (via (at 198.431686 125.533686) (size 0.8) (drill 0.4) (layers "F.Cu" "B.Cu") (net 10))
 (segment (start 202.747767 71.355) (end 200.442767 73.66) (width 0.4) (layer "B.Cu") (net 10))
 (segment (start 199.39 73.66) (end 198.12 74.93) (width 0.4) (layer "B.Cu") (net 10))
 (segment (start 189.16 83.89) (end 189.16 121.676944) (width 0.4) (layer "B.Cu") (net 10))
 (segment (start 192.197056 124.714) (end 197.612 124.714) (width 0.4) (layer "B.Cu") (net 10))
 (segment (start 200.442767 73.66) (end 199.39 73.66) (width 0.4) (layer "B.Cu") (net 10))
 (segment (start 198.12 74.93) (end 189.16 83.89) (width 0.4) (layer "B.Cu") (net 10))
 (segment (start 197.612 124.714) (end 198.431686 125.533686) (width 0.4) (layer "B.Cu") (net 10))
 (segment (start 203.52 71.355) (end 202.747767 71.355) (width 0.4) (layer "B.Cu") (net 10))
 (segment (start 189.16 121.676944) (end 192.197056 124.714) (width 0.4) (layer "B.Cu") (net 10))
 (segment (start 202.985 72.605) (end 200.66 74.93) (width 0.4) (layer "B.Cu") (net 11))
 (segment (start 192.283584 123.952) (end 198.374 123.952) (width 0.4) (layer "B.Cu") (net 11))
 (segment (start 206.06 71.355) (end 204.81 72.605) (width 0.4) (layer "B.Cu") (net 11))
 (segment (start 199.3925 124.9705) (end 199.3925 128.505) (width 0.4) (layer "B.Cu") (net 11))
 (segment (start 198.374 123.952) (end 199.3925 124.9705) (width 0.4) (layer "B.Cu") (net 11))
 (segment (start 191.7 83.89) (end 191.7 123.368416) (width 0.4) (layer "B.Cu") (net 11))
 (segment (start 204.81 72.605) (end 202.985 72.605) (width 0.4) (layer "B.Cu") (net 11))
 (segment (start 191.7 123.368416) (end 192.283584 123.952) (width 0.4) (layer "B.Cu") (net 11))
 (segment (start 200.66 74.93) (end 191.7 83.89) (width 0.4) (layer "B.Cu") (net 11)))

